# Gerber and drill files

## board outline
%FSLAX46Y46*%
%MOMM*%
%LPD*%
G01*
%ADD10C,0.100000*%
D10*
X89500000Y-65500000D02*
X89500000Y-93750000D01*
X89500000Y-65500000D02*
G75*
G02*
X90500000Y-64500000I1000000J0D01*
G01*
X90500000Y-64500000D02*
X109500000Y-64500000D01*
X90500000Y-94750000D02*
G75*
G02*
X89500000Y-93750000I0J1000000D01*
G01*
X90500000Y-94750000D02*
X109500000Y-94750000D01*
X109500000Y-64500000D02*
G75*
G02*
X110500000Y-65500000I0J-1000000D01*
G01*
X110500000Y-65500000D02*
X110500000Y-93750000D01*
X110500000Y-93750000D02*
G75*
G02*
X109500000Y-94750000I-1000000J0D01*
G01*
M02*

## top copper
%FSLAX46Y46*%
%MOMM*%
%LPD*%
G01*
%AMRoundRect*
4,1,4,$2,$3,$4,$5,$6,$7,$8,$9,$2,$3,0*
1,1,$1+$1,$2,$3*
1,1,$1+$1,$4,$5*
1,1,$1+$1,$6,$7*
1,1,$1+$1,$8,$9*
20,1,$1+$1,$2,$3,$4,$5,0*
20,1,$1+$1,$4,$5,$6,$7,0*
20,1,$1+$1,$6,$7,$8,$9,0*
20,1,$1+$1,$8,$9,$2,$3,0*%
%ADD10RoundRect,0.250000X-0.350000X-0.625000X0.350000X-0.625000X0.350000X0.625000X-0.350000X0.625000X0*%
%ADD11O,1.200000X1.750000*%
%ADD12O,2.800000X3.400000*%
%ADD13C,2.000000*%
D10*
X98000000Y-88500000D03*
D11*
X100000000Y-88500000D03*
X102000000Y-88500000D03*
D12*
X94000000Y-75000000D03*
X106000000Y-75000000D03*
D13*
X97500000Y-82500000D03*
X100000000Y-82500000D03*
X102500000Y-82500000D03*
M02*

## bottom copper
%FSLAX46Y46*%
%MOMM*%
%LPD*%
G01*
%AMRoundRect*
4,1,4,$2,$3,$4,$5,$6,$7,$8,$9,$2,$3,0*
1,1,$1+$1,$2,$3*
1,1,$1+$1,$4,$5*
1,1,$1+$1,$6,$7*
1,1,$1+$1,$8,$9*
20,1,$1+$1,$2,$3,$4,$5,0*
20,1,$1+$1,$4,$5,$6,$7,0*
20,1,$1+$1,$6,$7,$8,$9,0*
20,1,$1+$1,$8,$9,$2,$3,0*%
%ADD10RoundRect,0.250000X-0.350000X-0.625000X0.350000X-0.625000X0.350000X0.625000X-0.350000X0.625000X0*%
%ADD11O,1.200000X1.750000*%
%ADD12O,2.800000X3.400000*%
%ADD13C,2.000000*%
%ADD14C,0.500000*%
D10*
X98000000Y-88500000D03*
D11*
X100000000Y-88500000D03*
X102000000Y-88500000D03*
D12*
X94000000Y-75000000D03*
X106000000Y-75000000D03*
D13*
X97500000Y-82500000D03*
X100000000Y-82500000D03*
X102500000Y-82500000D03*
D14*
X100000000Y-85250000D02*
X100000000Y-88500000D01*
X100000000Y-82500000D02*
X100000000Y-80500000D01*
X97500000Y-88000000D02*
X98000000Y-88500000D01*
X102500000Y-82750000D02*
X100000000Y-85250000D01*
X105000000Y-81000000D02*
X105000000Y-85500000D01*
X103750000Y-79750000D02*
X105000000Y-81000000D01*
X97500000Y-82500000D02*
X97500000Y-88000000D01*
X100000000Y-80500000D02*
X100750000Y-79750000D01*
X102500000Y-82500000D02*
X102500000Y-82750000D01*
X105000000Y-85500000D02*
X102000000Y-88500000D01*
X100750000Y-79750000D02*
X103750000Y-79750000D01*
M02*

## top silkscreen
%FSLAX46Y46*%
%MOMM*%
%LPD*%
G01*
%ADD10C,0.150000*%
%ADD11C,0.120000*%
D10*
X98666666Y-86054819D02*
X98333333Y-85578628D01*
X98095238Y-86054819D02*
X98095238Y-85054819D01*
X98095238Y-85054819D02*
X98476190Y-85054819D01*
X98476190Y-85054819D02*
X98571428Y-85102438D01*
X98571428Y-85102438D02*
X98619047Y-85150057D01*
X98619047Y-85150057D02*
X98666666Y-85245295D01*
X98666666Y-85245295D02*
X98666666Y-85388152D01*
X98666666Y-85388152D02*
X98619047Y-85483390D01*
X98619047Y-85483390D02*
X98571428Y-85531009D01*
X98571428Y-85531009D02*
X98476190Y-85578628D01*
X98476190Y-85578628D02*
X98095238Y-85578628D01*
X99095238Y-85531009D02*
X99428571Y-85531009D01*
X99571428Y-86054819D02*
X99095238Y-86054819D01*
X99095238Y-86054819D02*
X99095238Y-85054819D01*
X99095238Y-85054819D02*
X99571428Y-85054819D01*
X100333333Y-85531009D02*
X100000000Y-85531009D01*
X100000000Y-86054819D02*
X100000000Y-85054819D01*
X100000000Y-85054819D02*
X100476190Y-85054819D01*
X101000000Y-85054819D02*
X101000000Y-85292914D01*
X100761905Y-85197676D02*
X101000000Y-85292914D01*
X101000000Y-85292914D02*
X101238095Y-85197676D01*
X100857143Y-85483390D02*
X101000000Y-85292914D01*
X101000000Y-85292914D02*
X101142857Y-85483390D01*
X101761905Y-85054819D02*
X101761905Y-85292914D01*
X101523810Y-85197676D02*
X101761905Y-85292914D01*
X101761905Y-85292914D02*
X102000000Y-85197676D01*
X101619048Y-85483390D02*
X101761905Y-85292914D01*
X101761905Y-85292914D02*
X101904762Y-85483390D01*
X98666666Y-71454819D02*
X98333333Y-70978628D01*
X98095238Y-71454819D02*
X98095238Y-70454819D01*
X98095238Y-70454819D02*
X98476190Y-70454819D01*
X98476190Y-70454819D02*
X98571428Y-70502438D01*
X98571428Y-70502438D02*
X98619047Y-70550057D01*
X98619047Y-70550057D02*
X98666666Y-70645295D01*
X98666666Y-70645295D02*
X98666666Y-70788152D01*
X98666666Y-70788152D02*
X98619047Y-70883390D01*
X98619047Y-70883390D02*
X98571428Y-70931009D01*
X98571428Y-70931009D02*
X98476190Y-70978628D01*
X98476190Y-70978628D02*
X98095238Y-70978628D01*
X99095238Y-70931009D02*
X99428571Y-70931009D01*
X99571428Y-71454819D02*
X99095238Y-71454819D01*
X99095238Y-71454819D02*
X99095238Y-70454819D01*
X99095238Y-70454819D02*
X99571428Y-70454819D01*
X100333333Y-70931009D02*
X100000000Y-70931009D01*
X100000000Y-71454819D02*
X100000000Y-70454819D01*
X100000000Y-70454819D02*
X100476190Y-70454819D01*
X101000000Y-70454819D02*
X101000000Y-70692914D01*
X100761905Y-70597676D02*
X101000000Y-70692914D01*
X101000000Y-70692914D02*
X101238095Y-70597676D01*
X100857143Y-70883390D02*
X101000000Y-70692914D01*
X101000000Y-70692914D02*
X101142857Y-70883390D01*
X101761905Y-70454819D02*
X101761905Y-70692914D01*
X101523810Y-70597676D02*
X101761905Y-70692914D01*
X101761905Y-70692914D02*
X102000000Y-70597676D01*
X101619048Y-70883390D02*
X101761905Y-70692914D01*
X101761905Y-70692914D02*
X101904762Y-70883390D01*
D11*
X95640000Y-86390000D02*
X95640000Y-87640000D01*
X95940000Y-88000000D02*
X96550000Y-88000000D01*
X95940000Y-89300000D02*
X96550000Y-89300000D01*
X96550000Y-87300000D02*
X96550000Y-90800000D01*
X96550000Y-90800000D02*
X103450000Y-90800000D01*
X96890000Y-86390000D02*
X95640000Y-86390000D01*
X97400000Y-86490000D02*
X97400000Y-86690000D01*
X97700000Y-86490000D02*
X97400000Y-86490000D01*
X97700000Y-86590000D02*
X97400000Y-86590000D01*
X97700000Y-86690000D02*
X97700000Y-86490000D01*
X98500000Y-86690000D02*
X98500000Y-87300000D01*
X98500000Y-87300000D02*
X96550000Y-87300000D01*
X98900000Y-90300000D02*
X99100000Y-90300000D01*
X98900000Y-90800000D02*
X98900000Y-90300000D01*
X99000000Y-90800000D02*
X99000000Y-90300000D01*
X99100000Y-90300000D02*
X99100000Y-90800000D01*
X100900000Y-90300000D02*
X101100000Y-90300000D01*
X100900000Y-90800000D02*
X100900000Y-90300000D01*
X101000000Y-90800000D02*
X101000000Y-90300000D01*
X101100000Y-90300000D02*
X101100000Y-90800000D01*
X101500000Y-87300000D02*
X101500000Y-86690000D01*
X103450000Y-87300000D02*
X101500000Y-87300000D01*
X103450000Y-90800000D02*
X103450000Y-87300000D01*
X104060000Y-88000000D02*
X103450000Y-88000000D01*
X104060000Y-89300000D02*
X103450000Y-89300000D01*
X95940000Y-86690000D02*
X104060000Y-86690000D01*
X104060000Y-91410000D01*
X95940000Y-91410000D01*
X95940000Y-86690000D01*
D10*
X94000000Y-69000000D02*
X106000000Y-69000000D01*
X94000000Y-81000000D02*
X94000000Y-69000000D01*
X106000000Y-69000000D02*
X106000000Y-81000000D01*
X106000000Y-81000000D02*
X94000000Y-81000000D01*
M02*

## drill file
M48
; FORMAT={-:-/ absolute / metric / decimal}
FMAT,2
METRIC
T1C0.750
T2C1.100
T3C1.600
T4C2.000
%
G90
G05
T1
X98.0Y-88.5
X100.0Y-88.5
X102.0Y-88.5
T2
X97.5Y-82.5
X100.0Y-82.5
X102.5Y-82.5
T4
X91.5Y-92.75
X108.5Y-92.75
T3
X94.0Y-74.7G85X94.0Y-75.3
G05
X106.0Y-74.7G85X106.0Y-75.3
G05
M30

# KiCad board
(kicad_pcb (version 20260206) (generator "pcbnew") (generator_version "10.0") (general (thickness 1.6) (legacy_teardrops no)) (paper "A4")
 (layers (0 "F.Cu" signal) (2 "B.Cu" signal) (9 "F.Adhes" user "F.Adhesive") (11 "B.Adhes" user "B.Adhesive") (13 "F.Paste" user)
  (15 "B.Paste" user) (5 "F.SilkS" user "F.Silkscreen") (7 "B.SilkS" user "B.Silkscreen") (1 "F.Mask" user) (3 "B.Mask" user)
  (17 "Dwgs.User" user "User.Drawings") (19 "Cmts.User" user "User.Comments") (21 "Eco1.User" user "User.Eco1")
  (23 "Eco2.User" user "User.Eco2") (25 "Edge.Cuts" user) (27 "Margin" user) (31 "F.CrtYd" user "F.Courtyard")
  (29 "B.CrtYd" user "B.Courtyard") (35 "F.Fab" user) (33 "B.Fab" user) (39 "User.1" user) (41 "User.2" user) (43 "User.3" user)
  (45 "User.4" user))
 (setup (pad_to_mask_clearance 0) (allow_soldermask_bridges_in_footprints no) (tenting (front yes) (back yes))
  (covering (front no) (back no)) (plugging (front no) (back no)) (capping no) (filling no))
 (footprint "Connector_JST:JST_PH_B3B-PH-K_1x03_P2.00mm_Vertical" (layer "F.Cu") (at 98 88.5)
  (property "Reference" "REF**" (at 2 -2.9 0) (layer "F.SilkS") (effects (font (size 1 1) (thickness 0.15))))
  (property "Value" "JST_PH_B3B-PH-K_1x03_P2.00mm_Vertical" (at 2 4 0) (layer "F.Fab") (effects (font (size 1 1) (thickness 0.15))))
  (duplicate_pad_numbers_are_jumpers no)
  (fp_line (start -2.36 -2.11) (end -2.36 -0.86) (stroke (width 0.12) (type solid)) (layer "F.SilkS"))
  (fp_line (start -2.06 -0.5) (end -1.45 -0.5) (stroke (width 0.12) (type solid)) (layer "F.SilkS"))
  (fp_line (start -2.06 0.8) (end -1.45 0.8) (stroke (width 0.12) (type solid)) (layer "F.SilkS"))
  (fp_line (start -1.45 -1.2) (end -1.45 2.3) (stroke (width 0.12) (type solid)) (layer "F.SilkS"))
  (fp_line (start -1.45 2.3) (end 5.45 2.3) (stroke (width 0.12) (type solid)) (layer "F.SilkS"))
  (fp_line (start -1.11 -2.11) (end -2.36 -2.11) (stroke (width 0.12) (type solid)) (layer "F.SilkS"))
  (fp_line (start -0.6 -2.01) (end -0.6 -1.81) (stroke (width 0.12) (type solid)) (layer "F.SilkS"))
  (fp_line (start -0.3 -2.01) (end -0.6 -2.01) (stroke (width 0.12) (type solid)) (layer "F.SilkS"))
  (fp_line (start -0.3 -1.91) (end -0.6 -1.91) (stroke (width 0.12) (type solid)) (layer "F.SilkS"))
  (fp_line (start -0.3 -1.81) (end -0.3 -2.01) (stroke (width 0.12) (type solid)) (layer "F.SilkS"))
  (fp_line (start 0.5 -1.81) (end 0.5 -1.2) (stroke (width 0.12) (type solid)) (layer "F.SilkS"))
  (fp_line (start 0.5 -1.2) (end -1.45 -1.2) (stroke (width 0.12) (type solid)) (layer "F.SilkS"))
  (fp_line (start 0.9 1.8) (end 1.1 1.8) (stroke (width 0.12) (type solid)) (layer "F.SilkS"))
  (fp_line (start 0.9 2.3) (end 0.9 1.8) (stroke (width 0.12) (type solid)) (layer "F.SilkS"))
  (fp_line (start 1 2.3) (end 1 1.8) (stroke (width 0.12) (type solid)) (layer "F.SilkS"))
  (fp_line (start 1.1 1.8) (end 1.1 2.3) (stroke (width 0.12) (type solid)) (layer "F.SilkS"))
  (fp_line (start 2.9 1.8) (end 3.1 1.8) (stroke (width 0.12) (type solid)) (layer "F.SilkS"))
  (fp_line (start 2.9 2.3) (end 2.9 1.8) (stroke (width 0.12) (type solid)) (layer "F.SilkS"))
  (fp_line (start 3 2.3) (end 3 1.8) (stroke (width 0.12) (type solid)) (layer "F.SilkS"))
  (fp_line (start 3.1 1.8) (end 3.1 2.3) (stroke (width 0.12) (type solid)) (layer "F.SilkS"))
  (fp_line (start 3.5 -1.2) (end 3.5 -1.81) (stroke (width 0.12) (type solid)) (layer "F.SilkS"))
  (fp_line (start 5.45 -1.2) (end 3.5 -1.2) (stroke (width 0.12) (type solid)) (layer "F.SilkS"))
  (fp_line (start 5.45 2.3) (end 5.45 -1.2) (stroke (width 0.12) (type solid)) (layer "F.SilkS"))
  (fp_line (start 6.06 -0.5) (end 5.45 -0.5) (stroke (width 0.12) (type solid)) (layer "F.SilkS"))
  (fp_line (start 6.06 0.8) (end 5.45 0.8) (stroke (width 0.12) (type solid)) (layer "F.SilkS"))
  (fp_rect (start -2.06 -1.81) (end 6.06 2.91) (stroke (width 0.12) (type solid)) (fill no) (layer "F.SilkS"))
  (pad "1" thru_hole roundrect (at 0 0) (size 1.2 1.75) (drill 0.75) (layers "*.Cu" "*.Mask") (remove_unused_layers no)
   (roundrect_rratio 0.208333))
  (pad "2" thru_hole oval (at 2 0) (size 1.2 1.75) (drill 0.75) (layers "*.Cu" "*.Mask") (remove_unused_layers no))
  (pad "3" thru_hole oval (at 4 0) (size 1.2 1.75) (drill 0.75) (layers "*.Cu" "*.Mask") (remove_unused_layers no)))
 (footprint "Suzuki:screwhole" (layer "F.Cu") (at 108.75 92.75)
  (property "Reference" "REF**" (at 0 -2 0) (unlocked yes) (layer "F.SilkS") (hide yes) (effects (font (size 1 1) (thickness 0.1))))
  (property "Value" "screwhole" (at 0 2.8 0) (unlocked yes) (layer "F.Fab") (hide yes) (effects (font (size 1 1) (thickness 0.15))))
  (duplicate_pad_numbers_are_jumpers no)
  (pad "" np_thru_hole circle (at -0.25 0) (size 2 2) (drill 2) (layers "*.Cu" "*.Mask")))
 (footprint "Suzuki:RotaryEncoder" (layer "F.Cu") (at 100 75)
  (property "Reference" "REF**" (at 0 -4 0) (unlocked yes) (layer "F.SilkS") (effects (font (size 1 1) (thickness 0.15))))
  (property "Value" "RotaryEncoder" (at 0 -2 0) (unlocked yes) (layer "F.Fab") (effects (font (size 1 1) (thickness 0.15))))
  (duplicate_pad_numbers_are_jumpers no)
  (fp_line (start -6 -6) (end 6 -6) (stroke (width 0.15) (type solid)) (layer "F.SilkS"))
  (fp_line (start -6 6) (end -6 -6) (stroke (width 0.15) (type solid)) (layer "F.SilkS"))
  (fp_line (start 6 -6) (end 6 6) (stroke (width 0.15) (type solid)) (layer "F.SilkS"))
  (fp_line (start 6 6) (end -6 6) (stroke (width 0.15) (type solid)) (layer "F.SilkS"))
  (pad "" thru_hole oval (at -6 0) (size 2.8 3.4) (drill oval 1.6 2.2) (layers "*.Cu" "*.Mask") (remove_unused_layers no)
   (thermal_bridge_angle 45))
  (pad "" thru_hole oval (at 6 0) (size 2.8 3.4) (drill oval 1.6 2.2) (layers "*.Cu" "*.Mask") (remove_unused_layers no)
   (thermal_bridge_angle 45))
  (pad "1" thru_hole circle (at -2.5 7.5) (size 2 2) (drill 1.1) (layers "*.Cu" "*.Mask") (remove_unused_layers no))
  (pad "2" thru_hole circle (at 0 7.5) (size 2 2) (drill 1.1) (layers "*.Cu" "*.Mask") (remove_unused_layers no))
  (pad "3" thru_hole circle (at 2.5 7.5) (size 2 2) (drill 1.1) (layers "*.Cu" "*.Mask") (remove_unused_layers no)))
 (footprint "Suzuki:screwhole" (layer "F.Cu") (at 91.5 92.75)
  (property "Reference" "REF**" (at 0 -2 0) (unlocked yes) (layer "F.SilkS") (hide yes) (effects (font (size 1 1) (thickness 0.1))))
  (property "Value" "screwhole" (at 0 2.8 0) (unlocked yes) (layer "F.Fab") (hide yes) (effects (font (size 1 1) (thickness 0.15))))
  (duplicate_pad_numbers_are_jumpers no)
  (pad "" np_thru_hole circle (at 0 0) (size 2 2) (drill 2) (layers "*.Cu" "*.Mask")))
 (gr_line (start 89.5 65.5) (end 89.5 93.75) (stroke (width 0.1) (type solid)) (layer "Edge.Cuts"))
 (gr_arc (start 89.5 65.5) (mid 89.792893 64.792893) (end 90.5 64.5) (stroke (width 0.1) (type default)) (layer "Edge.Cuts"))
 (gr_line (start 90.5 64.5) (end 109.5 64.5) (stroke (width 0.1) (type solid)) (layer "Edge.Cuts"))
 (gr_arc (start 90.5 94.75) (mid 89.792893 94.457107) (end 89.5 93.75) (stroke (width 0.1) (type default)) (layer "Edge.Cuts"))
 (gr_line (start 90.5 94.75) (end 109.5 94.75) (stroke (width 0.1) (type solid)) (layer "Edge.Cuts"))
 (gr_arc (start 109.5 64.5) (mid 110.207107 64.792893) (end 110.5 65.5) (stroke (width 0.1) (type default)) (layer "Edge.Cuts"))
 (gr_line (start 110.5 65.5) (end 110.5 93.75) (stroke (width 0.1) (type solid)) (layer "Edge.Cuts"))
 (gr_arc (start 110.5 93.75) (mid 110.207107 94.457107) (end 109.5 94.75) (stroke (width 0.1) (type default)) (layer "Edge.Cuts"))
 (segment (start 100 85.25) (end 100 88.5) (width 0.5) (layer "B.Cu") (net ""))
 (segment (start 100 82.5) (end 100 80.5) (width 0.5) (layer "B.Cu") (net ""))
 (segment (start 97.5 88) (end 98 88.5) (width 0.5) (layer "B.Cu") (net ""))
 (segment (start 102.5 82.75) (end 100 85.25) (width 0.5) (layer "B.Cu") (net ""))
 (segment (start 105 81) (end 105 85.5) (width 0.5) (layer "B.Cu") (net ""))
 (segment (start 103.75 79.75) (end 105 81) (width 0.5) (layer "B.Cu") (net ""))
 (segment (start 97.5 82.5) (end 97.5 88) (width 0.5) (layer "B.Cu") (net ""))
 (segment (start 100 80.5) (end 100.75 79.75) (width 0.5) (layer "B.Cu") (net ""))
 (segment (start 102.5 82.5) (end 102.5 82.75) (width 0.5) (layer "B.Cu") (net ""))
 (segment (start 105 85.5) (end 102 88.5) (width 0.5) (layer "B.Cu") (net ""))
 (segment (start 100.75 79.75) (end 103.75 79.75) (width 0.5) (layer "B.Cu") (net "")))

